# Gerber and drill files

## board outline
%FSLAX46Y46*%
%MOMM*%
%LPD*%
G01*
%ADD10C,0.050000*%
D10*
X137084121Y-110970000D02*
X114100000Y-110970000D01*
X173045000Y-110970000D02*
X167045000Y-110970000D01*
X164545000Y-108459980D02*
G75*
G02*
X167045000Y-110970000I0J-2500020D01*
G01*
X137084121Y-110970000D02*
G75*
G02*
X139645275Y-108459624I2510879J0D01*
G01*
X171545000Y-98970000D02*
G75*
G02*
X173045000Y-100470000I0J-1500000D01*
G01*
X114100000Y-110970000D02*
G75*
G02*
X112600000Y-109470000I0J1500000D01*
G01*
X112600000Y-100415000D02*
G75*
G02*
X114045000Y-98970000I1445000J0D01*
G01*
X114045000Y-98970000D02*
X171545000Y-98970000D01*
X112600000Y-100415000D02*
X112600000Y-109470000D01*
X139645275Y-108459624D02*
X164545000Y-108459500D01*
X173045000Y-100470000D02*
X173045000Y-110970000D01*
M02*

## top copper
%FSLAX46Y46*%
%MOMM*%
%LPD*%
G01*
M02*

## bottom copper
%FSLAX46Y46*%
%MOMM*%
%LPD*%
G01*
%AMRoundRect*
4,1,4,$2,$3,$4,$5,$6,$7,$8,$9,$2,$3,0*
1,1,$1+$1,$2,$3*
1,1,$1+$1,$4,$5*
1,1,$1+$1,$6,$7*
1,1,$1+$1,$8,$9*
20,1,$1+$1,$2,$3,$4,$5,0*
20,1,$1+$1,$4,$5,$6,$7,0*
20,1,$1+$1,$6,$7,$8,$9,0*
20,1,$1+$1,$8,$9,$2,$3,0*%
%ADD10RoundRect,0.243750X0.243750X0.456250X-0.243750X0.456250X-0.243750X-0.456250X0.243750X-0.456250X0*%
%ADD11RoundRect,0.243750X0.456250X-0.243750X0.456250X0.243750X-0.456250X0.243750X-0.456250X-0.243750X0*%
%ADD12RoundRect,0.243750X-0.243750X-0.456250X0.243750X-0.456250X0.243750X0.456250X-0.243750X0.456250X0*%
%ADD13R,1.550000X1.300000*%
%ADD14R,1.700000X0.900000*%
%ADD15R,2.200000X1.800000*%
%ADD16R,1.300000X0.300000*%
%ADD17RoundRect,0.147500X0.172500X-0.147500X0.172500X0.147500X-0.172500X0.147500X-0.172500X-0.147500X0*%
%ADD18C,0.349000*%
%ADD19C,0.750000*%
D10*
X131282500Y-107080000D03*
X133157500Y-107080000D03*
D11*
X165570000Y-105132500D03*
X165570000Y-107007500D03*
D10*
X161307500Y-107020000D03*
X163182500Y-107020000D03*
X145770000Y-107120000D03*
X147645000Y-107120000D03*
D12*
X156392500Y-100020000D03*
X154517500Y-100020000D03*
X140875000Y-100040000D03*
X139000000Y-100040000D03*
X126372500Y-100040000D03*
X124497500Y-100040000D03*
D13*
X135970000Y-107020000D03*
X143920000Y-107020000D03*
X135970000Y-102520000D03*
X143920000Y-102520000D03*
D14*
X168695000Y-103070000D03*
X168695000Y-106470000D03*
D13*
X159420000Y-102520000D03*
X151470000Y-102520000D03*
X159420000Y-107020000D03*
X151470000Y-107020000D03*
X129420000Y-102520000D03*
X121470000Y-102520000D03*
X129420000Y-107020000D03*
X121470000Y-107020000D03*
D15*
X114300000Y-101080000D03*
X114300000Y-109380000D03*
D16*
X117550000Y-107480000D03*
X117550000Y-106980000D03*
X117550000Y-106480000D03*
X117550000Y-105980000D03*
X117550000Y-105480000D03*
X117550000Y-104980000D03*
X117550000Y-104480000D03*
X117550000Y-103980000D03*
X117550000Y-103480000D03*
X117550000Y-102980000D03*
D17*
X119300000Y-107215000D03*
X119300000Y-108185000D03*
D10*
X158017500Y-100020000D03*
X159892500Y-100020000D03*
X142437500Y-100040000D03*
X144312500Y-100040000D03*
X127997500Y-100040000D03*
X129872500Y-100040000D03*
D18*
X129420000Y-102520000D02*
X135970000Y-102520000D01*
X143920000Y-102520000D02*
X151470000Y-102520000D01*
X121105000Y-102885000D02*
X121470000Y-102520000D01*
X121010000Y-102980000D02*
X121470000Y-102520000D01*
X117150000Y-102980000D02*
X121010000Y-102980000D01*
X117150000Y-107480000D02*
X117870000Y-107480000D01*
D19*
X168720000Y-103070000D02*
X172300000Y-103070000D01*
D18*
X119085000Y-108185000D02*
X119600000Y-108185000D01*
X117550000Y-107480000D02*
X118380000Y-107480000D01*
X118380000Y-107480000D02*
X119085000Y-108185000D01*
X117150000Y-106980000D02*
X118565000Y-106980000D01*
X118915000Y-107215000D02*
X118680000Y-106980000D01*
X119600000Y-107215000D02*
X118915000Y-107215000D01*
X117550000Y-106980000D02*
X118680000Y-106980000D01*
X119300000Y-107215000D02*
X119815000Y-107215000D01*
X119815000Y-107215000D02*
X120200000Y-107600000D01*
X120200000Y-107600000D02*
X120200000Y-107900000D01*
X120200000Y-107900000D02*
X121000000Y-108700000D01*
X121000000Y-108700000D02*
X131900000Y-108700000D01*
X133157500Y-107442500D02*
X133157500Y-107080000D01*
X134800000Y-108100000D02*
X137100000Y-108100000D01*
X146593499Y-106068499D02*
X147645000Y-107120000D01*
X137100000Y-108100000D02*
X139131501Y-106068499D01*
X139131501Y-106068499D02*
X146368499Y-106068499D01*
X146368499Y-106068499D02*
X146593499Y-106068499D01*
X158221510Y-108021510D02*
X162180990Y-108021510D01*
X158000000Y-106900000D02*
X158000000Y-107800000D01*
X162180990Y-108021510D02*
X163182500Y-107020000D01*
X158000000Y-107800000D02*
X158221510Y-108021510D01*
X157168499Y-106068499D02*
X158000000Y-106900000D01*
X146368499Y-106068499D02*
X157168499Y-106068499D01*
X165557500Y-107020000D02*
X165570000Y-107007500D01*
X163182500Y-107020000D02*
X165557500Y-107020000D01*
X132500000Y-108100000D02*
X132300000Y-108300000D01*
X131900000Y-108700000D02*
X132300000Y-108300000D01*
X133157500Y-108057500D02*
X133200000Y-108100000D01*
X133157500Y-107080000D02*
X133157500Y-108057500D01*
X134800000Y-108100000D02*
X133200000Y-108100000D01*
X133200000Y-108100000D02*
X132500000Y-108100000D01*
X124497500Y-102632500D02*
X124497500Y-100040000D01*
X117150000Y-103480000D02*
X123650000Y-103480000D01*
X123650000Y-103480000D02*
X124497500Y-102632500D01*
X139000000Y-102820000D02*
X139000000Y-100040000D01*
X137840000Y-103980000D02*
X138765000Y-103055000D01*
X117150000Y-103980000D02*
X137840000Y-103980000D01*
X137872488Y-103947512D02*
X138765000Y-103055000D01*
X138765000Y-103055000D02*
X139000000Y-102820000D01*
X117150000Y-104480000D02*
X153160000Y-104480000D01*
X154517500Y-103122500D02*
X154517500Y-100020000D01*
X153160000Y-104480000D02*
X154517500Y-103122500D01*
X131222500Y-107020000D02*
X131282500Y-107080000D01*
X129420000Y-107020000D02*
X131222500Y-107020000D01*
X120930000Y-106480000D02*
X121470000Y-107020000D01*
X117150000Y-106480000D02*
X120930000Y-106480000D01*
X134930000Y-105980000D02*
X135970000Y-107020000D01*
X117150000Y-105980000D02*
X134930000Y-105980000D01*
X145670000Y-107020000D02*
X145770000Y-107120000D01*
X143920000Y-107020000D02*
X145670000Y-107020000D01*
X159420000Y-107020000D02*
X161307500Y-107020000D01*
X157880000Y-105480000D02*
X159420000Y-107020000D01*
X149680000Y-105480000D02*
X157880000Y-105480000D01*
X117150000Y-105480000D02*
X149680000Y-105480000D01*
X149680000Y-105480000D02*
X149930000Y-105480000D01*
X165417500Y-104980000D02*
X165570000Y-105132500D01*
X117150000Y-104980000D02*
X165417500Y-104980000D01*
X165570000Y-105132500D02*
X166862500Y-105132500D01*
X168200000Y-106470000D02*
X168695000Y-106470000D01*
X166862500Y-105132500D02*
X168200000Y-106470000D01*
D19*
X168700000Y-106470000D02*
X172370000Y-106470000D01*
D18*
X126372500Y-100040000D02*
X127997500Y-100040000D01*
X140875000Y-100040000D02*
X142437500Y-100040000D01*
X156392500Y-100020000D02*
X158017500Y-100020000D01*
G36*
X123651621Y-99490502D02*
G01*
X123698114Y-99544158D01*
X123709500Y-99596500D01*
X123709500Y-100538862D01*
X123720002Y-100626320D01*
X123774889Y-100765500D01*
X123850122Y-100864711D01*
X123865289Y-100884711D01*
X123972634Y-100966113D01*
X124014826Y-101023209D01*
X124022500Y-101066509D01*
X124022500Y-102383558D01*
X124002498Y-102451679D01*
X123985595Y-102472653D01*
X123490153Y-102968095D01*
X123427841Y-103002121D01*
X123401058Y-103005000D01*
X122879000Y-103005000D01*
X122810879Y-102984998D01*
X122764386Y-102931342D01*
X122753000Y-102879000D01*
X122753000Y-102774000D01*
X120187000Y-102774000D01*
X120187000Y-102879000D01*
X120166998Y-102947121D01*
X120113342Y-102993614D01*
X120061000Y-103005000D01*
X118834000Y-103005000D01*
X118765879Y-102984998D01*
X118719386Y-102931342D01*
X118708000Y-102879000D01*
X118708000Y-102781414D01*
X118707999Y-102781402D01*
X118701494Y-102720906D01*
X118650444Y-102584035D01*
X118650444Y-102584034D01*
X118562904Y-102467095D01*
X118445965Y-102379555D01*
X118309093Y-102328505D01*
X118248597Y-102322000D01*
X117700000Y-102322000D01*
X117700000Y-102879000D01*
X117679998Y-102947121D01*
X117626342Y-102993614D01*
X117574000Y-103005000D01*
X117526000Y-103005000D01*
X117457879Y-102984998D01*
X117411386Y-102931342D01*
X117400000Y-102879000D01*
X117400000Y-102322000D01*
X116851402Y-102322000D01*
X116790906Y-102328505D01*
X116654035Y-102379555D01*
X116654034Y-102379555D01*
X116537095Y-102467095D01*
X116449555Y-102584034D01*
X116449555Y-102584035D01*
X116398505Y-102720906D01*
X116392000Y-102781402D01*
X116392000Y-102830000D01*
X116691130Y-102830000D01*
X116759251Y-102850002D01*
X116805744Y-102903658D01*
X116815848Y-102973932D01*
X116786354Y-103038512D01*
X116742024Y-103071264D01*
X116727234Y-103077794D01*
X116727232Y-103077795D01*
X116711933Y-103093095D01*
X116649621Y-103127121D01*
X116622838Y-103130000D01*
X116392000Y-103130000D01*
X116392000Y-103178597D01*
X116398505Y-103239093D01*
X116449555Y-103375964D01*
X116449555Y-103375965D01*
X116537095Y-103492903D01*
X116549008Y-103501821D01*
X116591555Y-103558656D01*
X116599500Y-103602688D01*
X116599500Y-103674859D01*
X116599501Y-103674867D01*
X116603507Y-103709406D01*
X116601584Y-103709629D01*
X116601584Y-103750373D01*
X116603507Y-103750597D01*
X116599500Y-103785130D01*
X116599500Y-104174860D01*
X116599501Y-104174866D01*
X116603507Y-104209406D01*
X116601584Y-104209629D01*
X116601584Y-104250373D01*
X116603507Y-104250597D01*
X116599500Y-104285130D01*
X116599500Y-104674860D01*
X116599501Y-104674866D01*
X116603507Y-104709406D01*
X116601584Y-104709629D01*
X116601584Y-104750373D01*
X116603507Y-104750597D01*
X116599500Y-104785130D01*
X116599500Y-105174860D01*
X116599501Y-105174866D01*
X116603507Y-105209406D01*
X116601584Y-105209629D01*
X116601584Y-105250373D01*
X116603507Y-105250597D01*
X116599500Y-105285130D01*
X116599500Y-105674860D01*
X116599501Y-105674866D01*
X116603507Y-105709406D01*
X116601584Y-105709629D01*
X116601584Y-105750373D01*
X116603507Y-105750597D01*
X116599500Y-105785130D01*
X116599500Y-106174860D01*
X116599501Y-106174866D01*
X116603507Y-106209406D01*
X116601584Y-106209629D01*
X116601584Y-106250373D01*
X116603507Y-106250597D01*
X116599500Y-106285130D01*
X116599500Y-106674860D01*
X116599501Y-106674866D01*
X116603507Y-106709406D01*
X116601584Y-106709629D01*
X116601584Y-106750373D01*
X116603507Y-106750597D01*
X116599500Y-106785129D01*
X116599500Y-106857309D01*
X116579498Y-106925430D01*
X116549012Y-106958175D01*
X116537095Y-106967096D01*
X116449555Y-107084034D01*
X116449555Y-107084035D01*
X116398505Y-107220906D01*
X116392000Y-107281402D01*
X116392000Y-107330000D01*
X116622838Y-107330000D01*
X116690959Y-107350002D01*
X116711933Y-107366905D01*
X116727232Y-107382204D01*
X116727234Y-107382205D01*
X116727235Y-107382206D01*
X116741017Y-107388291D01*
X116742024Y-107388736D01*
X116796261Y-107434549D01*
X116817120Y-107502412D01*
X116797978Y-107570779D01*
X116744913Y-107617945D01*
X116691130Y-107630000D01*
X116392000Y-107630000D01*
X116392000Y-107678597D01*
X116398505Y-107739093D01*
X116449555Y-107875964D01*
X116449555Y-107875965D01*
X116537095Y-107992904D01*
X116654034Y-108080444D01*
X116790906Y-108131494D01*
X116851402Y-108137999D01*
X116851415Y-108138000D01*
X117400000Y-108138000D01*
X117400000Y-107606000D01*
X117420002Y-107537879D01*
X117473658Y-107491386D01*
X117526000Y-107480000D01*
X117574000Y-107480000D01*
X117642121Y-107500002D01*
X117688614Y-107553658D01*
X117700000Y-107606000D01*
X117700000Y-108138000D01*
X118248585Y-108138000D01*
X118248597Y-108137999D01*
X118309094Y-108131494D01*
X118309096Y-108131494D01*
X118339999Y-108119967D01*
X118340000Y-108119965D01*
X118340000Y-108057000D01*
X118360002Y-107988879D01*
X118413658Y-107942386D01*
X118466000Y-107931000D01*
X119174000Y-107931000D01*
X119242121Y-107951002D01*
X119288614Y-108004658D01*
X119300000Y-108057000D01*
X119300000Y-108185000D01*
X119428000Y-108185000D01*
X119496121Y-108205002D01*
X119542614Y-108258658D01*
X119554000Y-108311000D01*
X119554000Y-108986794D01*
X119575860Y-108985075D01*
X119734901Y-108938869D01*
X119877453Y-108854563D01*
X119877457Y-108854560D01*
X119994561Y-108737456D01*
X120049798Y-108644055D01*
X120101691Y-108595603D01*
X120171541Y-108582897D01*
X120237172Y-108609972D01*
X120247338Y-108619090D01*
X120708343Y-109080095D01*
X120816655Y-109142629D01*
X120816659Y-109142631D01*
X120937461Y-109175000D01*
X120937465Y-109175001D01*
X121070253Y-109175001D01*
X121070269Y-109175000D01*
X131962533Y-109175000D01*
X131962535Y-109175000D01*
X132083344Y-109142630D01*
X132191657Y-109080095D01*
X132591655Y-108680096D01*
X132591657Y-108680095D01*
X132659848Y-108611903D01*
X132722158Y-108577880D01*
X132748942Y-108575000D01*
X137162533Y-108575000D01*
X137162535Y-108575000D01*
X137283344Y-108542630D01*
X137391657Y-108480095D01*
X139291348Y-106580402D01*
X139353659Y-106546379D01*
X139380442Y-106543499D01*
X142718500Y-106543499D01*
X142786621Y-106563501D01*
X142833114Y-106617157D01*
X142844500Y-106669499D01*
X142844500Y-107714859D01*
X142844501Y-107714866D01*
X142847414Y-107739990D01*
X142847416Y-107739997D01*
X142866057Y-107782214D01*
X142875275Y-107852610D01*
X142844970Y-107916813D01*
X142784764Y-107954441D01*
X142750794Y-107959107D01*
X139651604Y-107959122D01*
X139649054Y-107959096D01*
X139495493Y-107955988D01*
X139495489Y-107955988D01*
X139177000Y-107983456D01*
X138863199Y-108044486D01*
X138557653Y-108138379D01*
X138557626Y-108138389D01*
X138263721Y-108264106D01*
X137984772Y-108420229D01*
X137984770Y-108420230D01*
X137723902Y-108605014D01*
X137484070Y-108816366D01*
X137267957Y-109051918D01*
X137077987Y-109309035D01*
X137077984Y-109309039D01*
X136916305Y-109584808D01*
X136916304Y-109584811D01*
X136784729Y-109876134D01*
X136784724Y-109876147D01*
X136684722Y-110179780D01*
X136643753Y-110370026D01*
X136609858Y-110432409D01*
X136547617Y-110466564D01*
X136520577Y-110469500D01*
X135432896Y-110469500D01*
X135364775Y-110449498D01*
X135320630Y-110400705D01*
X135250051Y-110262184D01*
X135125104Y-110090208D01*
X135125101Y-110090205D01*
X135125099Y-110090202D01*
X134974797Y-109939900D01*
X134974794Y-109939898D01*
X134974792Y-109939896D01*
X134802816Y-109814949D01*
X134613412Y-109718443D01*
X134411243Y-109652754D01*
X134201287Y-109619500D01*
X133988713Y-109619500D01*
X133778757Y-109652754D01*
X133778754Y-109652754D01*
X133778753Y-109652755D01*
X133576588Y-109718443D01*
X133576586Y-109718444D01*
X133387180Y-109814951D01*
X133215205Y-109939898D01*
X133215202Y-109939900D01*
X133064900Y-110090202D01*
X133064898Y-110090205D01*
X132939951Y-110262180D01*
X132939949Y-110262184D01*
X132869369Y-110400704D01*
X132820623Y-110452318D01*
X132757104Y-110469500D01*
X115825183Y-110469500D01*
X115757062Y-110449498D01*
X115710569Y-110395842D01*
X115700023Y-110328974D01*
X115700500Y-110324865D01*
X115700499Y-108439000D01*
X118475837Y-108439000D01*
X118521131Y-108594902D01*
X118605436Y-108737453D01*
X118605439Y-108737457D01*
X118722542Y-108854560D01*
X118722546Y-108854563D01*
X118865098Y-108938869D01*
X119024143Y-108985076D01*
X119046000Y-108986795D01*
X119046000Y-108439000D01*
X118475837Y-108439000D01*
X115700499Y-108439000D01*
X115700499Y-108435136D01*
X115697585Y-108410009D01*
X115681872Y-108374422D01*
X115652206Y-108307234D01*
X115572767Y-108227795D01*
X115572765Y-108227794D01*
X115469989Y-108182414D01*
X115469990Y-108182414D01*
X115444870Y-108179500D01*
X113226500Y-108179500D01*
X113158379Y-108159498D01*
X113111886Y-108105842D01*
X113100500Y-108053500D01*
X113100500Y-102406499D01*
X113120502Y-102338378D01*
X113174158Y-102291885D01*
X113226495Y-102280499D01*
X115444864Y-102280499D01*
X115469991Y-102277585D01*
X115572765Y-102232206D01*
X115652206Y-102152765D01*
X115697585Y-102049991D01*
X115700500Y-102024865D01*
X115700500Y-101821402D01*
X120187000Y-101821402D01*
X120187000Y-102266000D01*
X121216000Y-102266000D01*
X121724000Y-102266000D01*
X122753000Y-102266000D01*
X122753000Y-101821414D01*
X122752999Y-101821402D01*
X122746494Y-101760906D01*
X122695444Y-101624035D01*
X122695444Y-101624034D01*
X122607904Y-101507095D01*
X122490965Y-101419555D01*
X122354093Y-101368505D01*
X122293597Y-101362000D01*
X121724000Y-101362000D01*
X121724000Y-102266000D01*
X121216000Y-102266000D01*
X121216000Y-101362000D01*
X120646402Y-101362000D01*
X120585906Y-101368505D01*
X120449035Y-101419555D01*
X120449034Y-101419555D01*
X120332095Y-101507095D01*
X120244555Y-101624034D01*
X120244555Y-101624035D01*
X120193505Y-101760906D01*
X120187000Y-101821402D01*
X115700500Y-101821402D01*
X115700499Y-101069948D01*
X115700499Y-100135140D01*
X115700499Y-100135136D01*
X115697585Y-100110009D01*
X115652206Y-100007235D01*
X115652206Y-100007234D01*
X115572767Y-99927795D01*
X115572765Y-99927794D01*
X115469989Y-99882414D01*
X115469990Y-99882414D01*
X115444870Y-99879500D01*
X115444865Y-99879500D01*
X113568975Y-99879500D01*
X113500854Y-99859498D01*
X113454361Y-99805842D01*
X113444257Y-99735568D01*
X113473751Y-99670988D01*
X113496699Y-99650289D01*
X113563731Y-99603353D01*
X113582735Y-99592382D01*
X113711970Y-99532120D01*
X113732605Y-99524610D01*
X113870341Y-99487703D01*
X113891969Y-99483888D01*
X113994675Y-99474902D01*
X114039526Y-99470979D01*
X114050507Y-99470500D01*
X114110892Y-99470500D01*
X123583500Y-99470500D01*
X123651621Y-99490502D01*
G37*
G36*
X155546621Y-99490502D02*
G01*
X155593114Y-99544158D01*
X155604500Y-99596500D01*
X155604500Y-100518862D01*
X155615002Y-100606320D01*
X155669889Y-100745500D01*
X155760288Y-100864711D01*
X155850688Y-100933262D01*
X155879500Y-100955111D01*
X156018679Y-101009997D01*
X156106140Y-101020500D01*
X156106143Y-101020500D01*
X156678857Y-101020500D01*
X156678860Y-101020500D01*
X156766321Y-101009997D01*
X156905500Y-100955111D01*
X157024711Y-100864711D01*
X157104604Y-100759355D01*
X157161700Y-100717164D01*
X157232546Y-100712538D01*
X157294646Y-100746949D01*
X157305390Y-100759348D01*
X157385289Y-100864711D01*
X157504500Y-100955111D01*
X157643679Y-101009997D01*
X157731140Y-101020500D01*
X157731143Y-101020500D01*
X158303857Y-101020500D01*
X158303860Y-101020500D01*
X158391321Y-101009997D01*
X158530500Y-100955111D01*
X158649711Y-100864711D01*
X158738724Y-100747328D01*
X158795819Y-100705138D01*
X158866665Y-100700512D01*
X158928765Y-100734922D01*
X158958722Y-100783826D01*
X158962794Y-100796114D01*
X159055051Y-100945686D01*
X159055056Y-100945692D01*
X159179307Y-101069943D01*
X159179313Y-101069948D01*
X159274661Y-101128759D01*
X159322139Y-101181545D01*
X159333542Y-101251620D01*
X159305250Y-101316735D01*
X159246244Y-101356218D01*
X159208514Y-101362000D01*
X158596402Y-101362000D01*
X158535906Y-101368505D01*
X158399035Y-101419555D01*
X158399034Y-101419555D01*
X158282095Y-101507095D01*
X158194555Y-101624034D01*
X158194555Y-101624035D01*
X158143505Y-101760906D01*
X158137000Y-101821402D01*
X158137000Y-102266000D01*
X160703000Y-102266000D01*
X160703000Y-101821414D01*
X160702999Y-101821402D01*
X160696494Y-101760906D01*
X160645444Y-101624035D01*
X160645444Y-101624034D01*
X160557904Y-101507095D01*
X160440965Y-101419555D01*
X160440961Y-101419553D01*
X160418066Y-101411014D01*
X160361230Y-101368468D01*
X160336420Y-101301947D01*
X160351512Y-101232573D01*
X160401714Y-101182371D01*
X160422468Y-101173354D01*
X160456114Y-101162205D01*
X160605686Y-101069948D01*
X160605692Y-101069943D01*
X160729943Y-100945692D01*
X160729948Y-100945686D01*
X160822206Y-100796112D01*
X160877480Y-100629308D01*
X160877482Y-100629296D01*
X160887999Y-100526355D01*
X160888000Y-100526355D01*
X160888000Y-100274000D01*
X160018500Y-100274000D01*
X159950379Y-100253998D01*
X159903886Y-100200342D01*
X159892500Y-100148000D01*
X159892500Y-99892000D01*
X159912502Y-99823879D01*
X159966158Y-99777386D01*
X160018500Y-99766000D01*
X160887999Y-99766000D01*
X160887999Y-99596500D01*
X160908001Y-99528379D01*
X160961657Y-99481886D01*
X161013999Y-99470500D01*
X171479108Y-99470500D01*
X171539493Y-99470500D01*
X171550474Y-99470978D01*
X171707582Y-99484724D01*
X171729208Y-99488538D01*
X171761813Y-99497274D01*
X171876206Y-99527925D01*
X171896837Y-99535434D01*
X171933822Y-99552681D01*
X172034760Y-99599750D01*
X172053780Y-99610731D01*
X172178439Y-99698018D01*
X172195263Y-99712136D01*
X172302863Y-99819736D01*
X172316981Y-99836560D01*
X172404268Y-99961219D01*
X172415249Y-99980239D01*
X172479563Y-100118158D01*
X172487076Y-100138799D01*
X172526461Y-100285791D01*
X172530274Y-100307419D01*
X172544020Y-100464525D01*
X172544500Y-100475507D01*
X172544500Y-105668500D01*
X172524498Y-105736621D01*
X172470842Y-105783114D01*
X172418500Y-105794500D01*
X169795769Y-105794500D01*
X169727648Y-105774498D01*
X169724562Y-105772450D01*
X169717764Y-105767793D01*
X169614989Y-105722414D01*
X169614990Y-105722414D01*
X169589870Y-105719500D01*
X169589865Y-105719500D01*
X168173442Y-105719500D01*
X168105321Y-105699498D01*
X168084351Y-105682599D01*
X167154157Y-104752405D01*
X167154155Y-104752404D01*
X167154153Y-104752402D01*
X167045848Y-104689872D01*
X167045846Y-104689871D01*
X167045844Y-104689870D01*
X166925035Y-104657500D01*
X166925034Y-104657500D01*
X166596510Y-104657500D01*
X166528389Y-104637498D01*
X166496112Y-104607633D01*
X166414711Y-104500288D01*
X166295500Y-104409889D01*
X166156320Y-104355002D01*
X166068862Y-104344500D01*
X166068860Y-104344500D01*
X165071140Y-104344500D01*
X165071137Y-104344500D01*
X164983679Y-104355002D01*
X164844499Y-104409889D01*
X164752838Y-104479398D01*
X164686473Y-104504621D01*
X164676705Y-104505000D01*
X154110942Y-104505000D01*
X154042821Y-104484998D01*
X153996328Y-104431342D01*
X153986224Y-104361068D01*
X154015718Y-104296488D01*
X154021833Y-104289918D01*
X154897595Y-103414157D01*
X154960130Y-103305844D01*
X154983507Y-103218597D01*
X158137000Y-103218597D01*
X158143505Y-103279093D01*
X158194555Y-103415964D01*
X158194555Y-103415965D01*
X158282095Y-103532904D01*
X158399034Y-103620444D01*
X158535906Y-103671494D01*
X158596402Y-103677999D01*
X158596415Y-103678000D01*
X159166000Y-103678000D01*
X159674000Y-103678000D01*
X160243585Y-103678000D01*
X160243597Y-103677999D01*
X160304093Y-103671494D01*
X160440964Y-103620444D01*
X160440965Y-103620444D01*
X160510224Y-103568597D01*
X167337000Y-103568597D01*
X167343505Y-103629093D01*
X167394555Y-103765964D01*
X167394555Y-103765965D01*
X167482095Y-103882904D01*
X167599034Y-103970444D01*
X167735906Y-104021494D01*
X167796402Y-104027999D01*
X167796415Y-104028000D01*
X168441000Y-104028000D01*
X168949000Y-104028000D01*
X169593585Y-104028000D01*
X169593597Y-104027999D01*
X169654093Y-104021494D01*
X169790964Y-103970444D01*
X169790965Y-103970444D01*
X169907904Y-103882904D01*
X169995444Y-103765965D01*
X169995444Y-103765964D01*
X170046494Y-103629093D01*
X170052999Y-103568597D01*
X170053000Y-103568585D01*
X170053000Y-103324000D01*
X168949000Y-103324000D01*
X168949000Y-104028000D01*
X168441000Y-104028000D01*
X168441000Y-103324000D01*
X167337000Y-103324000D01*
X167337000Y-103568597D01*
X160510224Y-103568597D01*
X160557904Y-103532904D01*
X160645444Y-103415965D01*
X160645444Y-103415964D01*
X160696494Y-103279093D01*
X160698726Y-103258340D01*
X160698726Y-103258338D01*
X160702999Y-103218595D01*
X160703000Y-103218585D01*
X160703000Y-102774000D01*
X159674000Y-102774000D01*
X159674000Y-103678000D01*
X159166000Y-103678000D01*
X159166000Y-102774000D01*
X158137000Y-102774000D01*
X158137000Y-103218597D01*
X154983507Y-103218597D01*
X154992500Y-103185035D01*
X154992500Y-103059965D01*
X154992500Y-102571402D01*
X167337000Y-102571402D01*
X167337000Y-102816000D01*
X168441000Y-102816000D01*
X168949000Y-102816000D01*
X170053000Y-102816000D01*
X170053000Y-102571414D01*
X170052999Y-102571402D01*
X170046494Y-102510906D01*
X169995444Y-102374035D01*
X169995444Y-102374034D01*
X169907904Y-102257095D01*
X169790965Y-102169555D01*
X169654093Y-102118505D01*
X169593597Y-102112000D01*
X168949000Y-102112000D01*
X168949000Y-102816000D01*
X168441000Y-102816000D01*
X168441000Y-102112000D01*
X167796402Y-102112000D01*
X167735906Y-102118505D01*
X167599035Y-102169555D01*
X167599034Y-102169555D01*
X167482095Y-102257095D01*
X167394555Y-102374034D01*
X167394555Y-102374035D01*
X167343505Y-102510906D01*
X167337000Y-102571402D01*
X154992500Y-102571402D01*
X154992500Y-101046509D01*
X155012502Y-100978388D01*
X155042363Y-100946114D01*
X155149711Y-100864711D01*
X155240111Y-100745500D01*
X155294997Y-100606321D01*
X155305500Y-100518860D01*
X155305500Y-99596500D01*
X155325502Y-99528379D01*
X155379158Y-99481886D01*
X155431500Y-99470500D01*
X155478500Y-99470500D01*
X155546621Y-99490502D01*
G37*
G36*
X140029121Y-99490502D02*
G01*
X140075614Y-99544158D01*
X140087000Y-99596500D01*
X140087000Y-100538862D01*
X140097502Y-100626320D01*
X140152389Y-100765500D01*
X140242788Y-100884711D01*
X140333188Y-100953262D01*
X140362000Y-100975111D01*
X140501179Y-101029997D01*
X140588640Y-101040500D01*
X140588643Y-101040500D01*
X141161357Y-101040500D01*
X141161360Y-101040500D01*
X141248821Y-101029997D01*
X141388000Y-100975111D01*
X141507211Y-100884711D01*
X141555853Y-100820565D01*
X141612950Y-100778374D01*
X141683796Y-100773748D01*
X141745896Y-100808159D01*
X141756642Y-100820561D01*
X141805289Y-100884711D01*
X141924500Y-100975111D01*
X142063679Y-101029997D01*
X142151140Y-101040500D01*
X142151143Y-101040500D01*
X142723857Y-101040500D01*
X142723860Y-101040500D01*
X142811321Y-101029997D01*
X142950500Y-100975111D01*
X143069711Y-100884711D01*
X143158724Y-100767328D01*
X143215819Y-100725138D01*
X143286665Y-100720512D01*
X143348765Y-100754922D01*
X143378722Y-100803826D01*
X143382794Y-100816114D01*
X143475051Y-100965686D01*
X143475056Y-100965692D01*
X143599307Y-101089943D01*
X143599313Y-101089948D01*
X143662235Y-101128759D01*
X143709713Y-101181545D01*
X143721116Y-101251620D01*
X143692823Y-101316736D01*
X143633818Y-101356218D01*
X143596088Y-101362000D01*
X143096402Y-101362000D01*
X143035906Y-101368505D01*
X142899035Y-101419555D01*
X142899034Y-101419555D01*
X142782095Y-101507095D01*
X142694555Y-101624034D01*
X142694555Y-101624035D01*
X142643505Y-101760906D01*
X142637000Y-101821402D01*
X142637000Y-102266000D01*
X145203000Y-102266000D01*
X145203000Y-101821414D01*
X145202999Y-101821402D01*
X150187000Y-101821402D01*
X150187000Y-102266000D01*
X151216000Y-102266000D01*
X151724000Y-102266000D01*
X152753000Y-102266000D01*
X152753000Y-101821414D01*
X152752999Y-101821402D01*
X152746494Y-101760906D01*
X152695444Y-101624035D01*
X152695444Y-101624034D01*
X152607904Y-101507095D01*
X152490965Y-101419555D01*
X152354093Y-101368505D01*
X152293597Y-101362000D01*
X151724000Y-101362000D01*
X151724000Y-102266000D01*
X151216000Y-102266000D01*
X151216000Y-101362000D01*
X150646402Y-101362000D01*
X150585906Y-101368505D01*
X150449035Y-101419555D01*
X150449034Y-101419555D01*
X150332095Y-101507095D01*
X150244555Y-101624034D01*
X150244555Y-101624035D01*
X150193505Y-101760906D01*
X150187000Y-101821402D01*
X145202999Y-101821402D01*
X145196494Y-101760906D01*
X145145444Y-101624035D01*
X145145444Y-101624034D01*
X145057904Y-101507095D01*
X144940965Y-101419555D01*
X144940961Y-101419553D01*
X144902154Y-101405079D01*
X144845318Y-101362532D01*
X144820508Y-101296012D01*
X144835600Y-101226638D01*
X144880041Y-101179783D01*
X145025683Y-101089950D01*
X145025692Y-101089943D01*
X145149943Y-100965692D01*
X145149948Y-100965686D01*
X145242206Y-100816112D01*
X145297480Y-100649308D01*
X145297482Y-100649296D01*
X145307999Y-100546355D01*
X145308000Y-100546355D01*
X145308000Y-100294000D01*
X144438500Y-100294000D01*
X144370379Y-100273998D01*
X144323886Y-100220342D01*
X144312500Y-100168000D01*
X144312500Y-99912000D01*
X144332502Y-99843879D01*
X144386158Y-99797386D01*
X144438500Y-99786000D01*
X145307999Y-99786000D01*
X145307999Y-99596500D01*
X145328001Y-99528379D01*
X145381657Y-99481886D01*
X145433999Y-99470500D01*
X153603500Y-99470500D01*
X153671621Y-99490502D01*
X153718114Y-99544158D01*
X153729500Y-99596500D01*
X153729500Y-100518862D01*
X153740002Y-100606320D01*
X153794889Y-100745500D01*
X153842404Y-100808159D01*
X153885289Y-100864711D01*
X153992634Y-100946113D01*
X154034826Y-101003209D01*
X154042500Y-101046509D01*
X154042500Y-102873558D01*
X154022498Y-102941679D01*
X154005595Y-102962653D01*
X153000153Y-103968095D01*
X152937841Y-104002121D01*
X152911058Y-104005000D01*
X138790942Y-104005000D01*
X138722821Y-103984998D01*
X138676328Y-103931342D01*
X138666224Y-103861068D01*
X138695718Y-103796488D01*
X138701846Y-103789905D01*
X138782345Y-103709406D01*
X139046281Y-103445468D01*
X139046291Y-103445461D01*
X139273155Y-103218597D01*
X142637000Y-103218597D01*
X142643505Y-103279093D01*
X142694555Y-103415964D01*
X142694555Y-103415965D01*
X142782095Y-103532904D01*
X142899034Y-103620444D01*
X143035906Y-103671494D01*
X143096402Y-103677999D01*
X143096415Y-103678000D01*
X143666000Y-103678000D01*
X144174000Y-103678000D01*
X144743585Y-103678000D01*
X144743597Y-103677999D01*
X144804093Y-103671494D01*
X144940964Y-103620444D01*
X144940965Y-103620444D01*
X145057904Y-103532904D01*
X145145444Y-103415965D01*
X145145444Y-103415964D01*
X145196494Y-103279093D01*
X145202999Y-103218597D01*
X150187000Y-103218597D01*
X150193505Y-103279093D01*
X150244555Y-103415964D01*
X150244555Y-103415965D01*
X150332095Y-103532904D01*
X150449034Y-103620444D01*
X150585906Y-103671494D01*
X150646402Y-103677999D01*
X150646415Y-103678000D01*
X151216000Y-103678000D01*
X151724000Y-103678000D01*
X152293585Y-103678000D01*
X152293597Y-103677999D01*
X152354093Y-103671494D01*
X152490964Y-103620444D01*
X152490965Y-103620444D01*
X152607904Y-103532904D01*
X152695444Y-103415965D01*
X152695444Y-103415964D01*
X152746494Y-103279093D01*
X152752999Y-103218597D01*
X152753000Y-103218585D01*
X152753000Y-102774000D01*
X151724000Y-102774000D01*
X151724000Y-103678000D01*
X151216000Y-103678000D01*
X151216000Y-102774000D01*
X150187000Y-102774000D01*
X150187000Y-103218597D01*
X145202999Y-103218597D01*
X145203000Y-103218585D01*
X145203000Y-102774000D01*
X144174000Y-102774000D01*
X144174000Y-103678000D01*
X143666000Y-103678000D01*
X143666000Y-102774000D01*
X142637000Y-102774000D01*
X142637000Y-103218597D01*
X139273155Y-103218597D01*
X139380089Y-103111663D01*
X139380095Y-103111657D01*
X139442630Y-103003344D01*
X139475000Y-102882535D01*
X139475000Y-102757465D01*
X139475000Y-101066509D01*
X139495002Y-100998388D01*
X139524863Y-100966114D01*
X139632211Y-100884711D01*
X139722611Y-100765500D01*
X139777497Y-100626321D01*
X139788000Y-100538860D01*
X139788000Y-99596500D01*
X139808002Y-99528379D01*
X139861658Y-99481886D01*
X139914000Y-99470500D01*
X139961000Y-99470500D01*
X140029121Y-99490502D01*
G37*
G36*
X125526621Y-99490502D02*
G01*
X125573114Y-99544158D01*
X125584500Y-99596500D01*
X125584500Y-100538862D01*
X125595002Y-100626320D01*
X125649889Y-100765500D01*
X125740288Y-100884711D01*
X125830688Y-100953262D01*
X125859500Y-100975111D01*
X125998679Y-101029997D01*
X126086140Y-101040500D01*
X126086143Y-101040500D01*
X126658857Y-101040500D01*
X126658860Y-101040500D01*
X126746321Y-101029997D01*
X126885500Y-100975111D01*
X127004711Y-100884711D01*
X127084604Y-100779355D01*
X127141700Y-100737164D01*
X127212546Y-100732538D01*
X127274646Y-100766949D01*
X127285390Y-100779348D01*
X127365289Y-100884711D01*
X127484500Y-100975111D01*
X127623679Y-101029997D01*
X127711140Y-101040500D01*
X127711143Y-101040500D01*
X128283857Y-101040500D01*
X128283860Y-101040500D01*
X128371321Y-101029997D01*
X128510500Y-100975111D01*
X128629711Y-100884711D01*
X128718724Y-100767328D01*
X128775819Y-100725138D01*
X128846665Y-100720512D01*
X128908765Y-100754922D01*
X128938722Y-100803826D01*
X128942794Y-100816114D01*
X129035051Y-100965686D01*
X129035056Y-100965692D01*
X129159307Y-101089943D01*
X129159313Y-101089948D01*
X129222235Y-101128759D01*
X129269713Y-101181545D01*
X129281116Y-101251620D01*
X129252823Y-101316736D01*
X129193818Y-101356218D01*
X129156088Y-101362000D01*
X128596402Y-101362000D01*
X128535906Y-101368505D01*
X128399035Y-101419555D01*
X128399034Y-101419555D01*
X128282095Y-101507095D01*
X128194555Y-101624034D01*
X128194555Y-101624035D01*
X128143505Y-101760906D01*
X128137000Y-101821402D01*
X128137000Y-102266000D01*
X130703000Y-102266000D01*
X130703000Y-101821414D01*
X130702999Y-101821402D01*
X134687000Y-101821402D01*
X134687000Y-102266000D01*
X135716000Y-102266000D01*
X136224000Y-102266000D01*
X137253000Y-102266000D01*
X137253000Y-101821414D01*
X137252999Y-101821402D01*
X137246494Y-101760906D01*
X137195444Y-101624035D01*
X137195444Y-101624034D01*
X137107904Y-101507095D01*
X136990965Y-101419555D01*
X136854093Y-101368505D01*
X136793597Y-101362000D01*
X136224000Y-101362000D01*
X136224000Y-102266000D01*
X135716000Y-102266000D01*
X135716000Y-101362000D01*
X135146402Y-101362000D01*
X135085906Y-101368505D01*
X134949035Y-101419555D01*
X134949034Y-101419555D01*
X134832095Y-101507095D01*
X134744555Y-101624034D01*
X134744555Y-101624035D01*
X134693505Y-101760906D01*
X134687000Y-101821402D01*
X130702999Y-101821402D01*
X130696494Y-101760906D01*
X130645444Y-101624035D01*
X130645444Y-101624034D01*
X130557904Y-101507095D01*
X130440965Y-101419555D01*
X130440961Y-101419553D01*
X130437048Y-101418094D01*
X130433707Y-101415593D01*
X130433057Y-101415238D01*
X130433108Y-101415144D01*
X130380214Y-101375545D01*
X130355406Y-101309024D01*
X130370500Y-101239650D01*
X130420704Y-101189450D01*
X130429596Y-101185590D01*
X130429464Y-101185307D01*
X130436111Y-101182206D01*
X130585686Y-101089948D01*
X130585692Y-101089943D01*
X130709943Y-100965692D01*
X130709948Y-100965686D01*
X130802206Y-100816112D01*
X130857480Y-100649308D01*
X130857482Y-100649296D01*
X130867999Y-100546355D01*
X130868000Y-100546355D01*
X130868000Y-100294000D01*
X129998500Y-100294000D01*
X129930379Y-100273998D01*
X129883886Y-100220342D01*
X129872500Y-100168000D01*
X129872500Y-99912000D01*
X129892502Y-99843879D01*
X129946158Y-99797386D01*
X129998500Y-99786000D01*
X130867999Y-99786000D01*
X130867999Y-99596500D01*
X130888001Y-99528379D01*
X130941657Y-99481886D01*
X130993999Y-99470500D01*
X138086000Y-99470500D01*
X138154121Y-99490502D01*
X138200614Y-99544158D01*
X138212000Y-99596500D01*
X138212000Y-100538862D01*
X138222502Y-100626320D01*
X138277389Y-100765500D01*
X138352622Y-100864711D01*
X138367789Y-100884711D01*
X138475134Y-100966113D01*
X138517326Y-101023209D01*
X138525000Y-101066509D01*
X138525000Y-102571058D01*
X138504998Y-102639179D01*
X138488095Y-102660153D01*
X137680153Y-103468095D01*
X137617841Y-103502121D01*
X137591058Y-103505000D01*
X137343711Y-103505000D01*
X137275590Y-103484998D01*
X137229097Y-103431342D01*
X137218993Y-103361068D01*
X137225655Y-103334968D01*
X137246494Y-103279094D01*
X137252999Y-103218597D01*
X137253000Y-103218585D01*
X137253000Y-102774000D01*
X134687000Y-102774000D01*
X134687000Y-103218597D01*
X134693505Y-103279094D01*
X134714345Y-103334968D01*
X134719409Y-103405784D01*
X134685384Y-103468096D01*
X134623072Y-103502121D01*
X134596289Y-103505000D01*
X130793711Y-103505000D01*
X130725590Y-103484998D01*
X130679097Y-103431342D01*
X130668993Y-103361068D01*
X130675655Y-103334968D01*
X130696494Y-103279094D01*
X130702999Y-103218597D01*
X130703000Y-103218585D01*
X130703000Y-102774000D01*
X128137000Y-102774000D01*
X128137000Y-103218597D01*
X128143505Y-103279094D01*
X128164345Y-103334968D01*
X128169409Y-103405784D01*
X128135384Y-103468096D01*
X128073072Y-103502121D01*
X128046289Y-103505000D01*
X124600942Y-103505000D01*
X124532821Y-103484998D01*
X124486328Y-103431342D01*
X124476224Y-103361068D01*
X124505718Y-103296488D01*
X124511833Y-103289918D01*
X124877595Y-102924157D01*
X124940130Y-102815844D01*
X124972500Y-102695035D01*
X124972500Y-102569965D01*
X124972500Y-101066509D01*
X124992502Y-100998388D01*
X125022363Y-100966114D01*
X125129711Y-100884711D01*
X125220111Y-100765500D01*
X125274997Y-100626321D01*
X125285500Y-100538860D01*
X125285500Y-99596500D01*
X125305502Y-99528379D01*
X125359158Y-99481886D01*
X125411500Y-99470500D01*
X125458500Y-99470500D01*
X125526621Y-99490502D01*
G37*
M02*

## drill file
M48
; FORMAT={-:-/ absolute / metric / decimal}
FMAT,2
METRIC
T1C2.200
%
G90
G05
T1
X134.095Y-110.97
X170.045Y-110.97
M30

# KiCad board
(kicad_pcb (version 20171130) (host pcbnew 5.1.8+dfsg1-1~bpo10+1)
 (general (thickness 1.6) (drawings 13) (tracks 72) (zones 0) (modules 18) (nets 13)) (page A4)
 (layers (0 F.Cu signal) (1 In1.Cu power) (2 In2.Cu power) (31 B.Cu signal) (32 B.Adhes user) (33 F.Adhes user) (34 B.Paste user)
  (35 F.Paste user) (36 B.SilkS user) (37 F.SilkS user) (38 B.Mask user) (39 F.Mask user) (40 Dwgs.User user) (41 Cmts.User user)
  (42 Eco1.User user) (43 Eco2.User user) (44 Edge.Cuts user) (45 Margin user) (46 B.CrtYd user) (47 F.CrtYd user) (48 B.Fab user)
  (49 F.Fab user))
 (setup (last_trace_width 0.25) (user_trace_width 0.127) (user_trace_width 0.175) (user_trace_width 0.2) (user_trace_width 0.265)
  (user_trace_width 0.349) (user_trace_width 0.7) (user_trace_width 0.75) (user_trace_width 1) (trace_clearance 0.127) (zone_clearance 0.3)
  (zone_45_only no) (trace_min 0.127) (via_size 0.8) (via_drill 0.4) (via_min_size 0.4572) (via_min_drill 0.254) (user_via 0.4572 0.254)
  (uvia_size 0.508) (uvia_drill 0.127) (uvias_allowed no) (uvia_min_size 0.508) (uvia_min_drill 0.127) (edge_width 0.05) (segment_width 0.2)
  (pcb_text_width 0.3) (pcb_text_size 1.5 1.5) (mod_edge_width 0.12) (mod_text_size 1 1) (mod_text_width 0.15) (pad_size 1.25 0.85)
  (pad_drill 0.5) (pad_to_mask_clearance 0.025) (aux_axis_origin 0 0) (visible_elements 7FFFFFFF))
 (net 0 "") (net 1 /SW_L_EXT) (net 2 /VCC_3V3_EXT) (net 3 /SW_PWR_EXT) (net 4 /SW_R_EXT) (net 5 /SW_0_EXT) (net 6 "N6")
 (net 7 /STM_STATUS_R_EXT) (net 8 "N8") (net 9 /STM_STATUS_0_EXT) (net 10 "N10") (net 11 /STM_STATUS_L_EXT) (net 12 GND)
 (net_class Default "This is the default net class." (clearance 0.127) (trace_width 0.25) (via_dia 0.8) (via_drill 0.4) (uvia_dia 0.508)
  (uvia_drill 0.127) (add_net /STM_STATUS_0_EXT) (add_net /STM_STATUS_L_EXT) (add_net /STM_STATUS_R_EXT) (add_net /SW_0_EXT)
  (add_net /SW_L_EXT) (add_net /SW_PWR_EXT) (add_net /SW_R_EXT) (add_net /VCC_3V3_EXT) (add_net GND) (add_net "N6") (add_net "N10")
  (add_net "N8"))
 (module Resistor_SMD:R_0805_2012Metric (layer B.Cu) (at 132.22 107.08 180)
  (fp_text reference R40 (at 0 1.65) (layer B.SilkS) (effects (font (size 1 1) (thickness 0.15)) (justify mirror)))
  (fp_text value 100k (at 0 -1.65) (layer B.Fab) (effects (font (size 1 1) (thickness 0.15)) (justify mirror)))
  (pad 2 smd roundrect (at 0.9375 0 180) (size 0.975 1.4) (layers B.Cu B.Paste B.Mask) (roundrect_rratio 0.25) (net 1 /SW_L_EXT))
  (pad 1 smd roundrect (at -0.9375 0 180) (size 0.975 1.4) (layers B.Cu B.Paste B.Mask) (roundrect_rratio 0.25) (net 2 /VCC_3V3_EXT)))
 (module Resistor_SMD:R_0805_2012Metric (layer B.Cu) (at 165.57 106.07 90)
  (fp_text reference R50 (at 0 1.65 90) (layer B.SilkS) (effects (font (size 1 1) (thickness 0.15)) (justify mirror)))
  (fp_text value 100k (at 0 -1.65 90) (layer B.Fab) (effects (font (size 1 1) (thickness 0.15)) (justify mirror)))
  (pad 2 smd roundrect (at 0.9375 0 90) (size 0.975 1.4) (layers B.Cu B.Paste B.Mask) (roundrect_rratio 0.25) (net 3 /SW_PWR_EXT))
  (pad 1 smd roundrect (at -0.9375 0 90) (size 0.975 1.4) (layers B.Cu B.Paste B.Mask) (roundrect_rratio 0.25) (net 2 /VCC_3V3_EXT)))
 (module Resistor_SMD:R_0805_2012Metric (layer B.Cu) (at 162.245 107.02 180)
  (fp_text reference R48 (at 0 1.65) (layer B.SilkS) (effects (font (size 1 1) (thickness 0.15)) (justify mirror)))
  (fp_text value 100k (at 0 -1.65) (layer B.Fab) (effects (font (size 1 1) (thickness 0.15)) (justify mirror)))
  (pad 2 smd roundrect (at 0.9375 0 180) (size 0.975 1.4) (layers B.Cu B.Paste B.Mask) (roundrect_rratio 0.25) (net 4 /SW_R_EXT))
  (pad 1 smd roundrect (at -0.9375 0 180) (size 0.975 1.4) (layers B.Cu B.Paste B.Mask) (roundrect_rratio 0.25) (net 2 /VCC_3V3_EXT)))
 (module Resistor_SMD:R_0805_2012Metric (layer B.Cu) (at 146.7075 107.12 180)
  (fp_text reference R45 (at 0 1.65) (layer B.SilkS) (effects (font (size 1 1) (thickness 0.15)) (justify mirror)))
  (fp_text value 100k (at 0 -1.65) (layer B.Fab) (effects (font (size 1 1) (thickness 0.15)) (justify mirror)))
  (pad 2 smd roundrect (at 0.9375 0 180) (size 0.975 1.4) (layers B.Cu B.Paste B.Mask) (roundrect_rratio 0.25) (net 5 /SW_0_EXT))
  (pad 1 smd roundrect (at -0.9375 0 180) (size 0.975 1.4) (layers B.Cu B.Paste B.Mask) (roundrect_rratio 0.25) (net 2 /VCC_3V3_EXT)))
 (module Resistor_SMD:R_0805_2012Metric (layer B.Cu) (at 155.455 100.02)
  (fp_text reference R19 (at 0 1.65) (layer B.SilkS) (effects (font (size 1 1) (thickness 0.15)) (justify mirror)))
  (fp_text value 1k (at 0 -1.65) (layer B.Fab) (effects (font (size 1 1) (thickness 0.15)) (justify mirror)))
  (pad 2 smd roundrect (at 0.9375 0) (size 0.975 1.4) (layers B.Cu B.Paste B.Mask) (roundrect_rratio 0.25) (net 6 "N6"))
  (pad 1 smd roundrect (at -0.9375 0) (size 0.975 1.4) (layers B.Cu B.Paste B.Mask) (roundrect_rratio 0.25) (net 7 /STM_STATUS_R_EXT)))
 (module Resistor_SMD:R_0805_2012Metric (layer B.Cu) (at 139.9375 100.04)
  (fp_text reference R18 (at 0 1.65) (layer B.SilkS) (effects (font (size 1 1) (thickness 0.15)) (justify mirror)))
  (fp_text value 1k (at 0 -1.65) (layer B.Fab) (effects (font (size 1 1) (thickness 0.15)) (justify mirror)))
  (pad 2 smd roundrect (at 0.9375 0) (size 0.975 1.4) (layers B.Cu B.Paste B.Mask) (roundrect_rratio 0.25) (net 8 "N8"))
  (pad 1 smd roundrect (at -0.9375 0) (size 0.975 1.4) (layers B.Cu B.Paste B.Mask) (roundrect_rratio 0.25) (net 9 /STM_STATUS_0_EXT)))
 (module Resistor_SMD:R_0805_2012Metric (layer B.Cu) (at 125.435 100.04)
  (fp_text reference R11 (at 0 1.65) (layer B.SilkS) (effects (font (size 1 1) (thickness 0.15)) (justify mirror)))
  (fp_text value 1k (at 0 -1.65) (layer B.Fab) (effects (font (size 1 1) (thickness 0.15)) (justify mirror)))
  (pad 2 smd roundrect (at 0.9375 0) (size 0.975 1.4) (layers B.Cu B.Paste B.Mask) (roundrect_rratio 0.25) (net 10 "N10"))
  (pad 1 smd roundrect (at -0.9375 0) (size 0.975 1.4) (layers B.Cu B.Paste B.Mask) (roundrect_rratio 0.25) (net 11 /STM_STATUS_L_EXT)))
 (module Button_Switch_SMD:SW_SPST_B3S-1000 (layer B.Cu) (at 139.945 104.77)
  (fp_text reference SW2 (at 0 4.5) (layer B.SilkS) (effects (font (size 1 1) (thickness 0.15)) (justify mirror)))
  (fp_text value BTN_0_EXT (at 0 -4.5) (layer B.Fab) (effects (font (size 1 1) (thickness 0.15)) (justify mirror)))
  (pad 1 smd rect (at -3.975 2.25) (size 1.55 1.3) (layers B.Cu B.Paste B.Mask) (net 5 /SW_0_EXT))
  (pad 1 smd rect (at 3.975 2.25) (size 1.55 1.3) (layers B.Cu B.Paste B.Mask) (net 5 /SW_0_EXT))
  (pad 2 smd rect (at -3.975 -2.25) (size 1.55 1.3) (layers B.Cu B.Paste B.Mask) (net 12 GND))
  (pad 2 smd rect (at 3.975 -2.25) (size 1.55 1.3) (layers B.Cu B.Paste B.Mask) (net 12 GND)))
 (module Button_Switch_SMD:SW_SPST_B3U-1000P (layer B.Cu) (at 168.695 104.77 90)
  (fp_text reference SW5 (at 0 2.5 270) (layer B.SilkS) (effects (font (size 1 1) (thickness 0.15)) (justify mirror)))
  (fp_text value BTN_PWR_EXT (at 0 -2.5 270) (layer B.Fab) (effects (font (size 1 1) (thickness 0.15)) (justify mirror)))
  (pad 2 smd rect (at 1.7 0 90) (size 0.9 1.7) (layers B.Cu B.Paste B.Mask) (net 12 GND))
  (pad 1 smd rect (at -1.7 0 90) (size 0.9 1.7) (layers B.Cu B.Paste B.Mask) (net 3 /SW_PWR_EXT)))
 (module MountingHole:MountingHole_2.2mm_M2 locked (layer F.Cu) (at 134.095 110.97 180)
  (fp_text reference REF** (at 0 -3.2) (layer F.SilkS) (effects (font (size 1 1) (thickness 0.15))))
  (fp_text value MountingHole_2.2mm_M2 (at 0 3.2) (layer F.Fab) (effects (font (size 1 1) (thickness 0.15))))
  (pad 1 np_thru_hole circle (at 0 0 180) (size 2.2 2.2) (drill 2.2) (layers *.Cu *.Mask)))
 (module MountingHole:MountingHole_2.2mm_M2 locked (layer F.Cu) (at 170.045 110.97 270)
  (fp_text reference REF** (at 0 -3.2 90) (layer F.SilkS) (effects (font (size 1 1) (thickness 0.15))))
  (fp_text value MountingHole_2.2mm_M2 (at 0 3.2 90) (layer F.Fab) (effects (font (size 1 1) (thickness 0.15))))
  (pad 1 np_thru_hole circle (at 0 0 270) (size 2.2 2.2) (drill 2.2) (layers *.Cu *.Mask)))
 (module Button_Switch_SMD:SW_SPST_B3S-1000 (layer B.Cu) (at 155.445 104.77)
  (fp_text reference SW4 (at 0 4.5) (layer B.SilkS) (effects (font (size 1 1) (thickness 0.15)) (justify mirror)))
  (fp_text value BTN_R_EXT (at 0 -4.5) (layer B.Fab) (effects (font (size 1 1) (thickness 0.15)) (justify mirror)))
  (pad 2 smd rect (at 3.975 -2.25) (size 1.55 1.3) (layers B.Cu B.Paste B.Mask) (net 12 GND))
  (pad 2 smd rect (at -3.975 -2.25) (size 1.55 1.3) (layers B.Cu B.Paste B.Mask) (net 12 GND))
  (pad 1 smd rect (at 3.975 2.25) (size 1.55 1.3) (layers B.Cu B.Paste B.Mask) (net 4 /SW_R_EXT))
  (pad 1 smd rect (at -3.975 2.25) (size 1.55 1.3) (layers B.Cu B.Paste B.Mask) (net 4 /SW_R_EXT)))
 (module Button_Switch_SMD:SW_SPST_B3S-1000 (layer B.Cu) (at 125.445 104.77)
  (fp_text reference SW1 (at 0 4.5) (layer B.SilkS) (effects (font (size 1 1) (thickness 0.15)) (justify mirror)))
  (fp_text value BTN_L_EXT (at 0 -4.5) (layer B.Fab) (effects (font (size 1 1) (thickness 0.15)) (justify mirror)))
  (pad 2 smd rect (at 3.975 -2.25) (size 1.55 1.3) (layers B.Cu B.Paste B.Mask) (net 12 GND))
  (pad 2 smd rect (at -3.975 -2.25) (size 1.55 1.3) (layers B.Cu B.Paste B.Mask) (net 12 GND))
  (pad 1 smd rect (at 3.975 2.25) (size 1.55 1.3) (layers B.Cu B.Paste B.Mask) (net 1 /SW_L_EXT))
  (pad 1 smd rect (at -3.975 2.25) (size 1.55 1.3) (layers B.Cu B.Paste B.Mask) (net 1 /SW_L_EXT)))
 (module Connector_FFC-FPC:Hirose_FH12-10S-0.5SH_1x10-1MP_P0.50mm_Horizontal (layer B.Cu) (at 115.7 105.23 90)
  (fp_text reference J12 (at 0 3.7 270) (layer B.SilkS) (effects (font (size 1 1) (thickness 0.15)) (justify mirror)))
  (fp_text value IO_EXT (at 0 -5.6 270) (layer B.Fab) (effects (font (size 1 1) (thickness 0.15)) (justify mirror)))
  (pad MP smd rect (at 4.15 -1.4 90) (size 1.8 2.2) (layers B.Cu B.Paste B.Mask))
  (pad MP smd rect (at -4.15 -1.4 90) (size 1.8 2.2) (layers B.Cu B.Paste B.Mask))
  (pad 1 smd rect (at -2.25 1.85 90) (size 0.3 1.3) (layers B.Cu B.Paste B.Mask) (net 12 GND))
  (pad 2 smd rect (at -1.75 1.85 90) (size 0.3 1.3) (layers B.Cu B.Paste B.Mask) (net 2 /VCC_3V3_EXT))
  (pad 3 smd rect (at -1.25 1.85 90) (size 0.3 1.3) (layers B.Cu B.Paste B.Mask) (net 1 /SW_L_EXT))
  (pad 4 smd rect (at -0.75 1.85 90) (size 0.3 1.3) (layers B.Cu B.Paste B.Mask) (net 5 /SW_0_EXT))
  (pad 5 smd rect (at -0.25 1.85 90) (size 0.3 1.3) (layers B.Cu B.Paste B.Mask) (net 4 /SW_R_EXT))
  (pad 6 smd rect (at 0.25 1.85 90) (size 0.3 1.3) (layers B.Cu B.Paste B.Mask) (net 3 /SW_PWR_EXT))
  (pad 7 smd rect (at 0.75 1.85 90) (size 0.3 1.3) (layers B.Cu B.Paste B.Mask) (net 7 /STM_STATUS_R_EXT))
  (pad 8 smd rect (at 1.25 1.85 90) (size 0.3 1.3) (layers B.Cu B.Paste B.Mask) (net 9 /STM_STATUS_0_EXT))
  (pad 9 smd rect (at 1.75 1.85 90) (size 0.3 1.3) (layers B.Cu B.Paste B.Mask) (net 11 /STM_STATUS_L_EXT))
  (pad 10 smd rect (at 2.25 1.85 90) (size 0.3 1.3) (layers B.Cu B.Paste B.Mask) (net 12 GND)))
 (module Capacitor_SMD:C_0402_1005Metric (layer B.Cu) (at 119.3 107.7 90)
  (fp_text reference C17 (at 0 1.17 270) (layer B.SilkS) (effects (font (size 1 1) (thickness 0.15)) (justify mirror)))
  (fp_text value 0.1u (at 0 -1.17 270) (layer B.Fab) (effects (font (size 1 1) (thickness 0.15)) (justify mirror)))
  (pad 2 smd roundrect (at 0.485 0 90) (size 0.59 0.64) (layers B.Cu B.Paste B.Mask) (roundrect_rratio 0.25) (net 2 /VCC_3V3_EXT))
  (pad 1 smd roundrect (at -0.485 0 90) (size 0.59 0.64) (layers B.Cu B.Paste B.Mask) (roundrect_rratio 0.25) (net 12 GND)))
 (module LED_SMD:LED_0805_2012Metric (layer B.Cu) (at 158.955 100.02 180)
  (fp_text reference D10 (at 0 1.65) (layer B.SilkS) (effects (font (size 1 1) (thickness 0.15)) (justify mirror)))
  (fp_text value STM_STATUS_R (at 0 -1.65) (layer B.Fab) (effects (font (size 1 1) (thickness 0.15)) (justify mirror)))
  (pad 2 smd roundrect (at 0.9375 0 180) (size 0.975 1.4) (layers B.Cu B.Paste B.Mask) (roundrect_rratio 0.25) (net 6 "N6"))
  (pad 1 smd roundrect (at -0.9375 0 180) (size 0.975 1.4) (layers B.Cu B.Paste B.Mask) (roundrect_rratio 0.25) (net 12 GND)))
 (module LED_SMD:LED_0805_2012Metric (layer B.Cu) (at 143.375 100.04 180)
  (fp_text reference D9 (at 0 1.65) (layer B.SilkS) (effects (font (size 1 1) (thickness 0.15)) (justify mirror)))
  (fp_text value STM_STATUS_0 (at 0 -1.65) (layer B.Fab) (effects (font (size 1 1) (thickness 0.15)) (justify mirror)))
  (pad 2 smd roundrect (at 0.9375 0 180) (size 0.975 1.4) (layers B.Cu B.Paste B.Mask) (roundrect_rratio 0.25) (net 8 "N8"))
  (pad 1 smd roundrect (at -0.9375 0 180) (size 0.975 1.4) (layers B.Cu B.Paste B.Mask) (roundrect_rratio 0.25) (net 12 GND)))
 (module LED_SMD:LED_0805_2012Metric (layer B.Cu) (at 128.935 100.04 180)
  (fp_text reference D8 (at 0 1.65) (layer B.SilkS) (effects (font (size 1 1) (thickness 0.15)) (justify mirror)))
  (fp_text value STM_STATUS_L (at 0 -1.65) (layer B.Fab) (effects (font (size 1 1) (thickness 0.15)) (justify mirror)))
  (pad 2 smd roundrect (at 0.9375 0 180) (size 0.975 1.4) (layers B.Cu B.Paste B.Mask) (roundrect_rratio 0.25) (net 10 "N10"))
  (pad 1 smd roundrect (at -0.9375 0 180) (size 0.975 1.4) (layers B.Cu B.Paste B.Mask) (roundrect_rratio 0.25) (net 12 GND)))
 (gr_line (start 137.084121 110.97) (end 114.1 110.97) (layer Edge.Cuts) (width 0.05))
 (gr_line (start 173.045 110.97) (end 167.045 110.97) (layer Edge.Cuts) (width 0.05))
 (gr_arc (start 164.545 110.96) (end 167.045 110.97) (angle -90.2291819) (layer Edge.Cuts) (width 0.05))
 (gr_arc (start 139.595 110.97) (end 137.084121 110.97) (angle 91.14730236) (layer Edge.Cuts) (width 0.05))
 (gr_arc (start 171.545 100.47) (end 173.045 100.47) (angle -90) (layer Edge.Cuts) (width 0.05))
 (gr_arc (start 114.1 109.47) (end 114.1 110.97) (angle 90) (layer Edge.Cuts) (width 0.05))
 (gr_arc (start 114.045 100.415) (end 112.6 100.415) (angle 90) (layer Edge.Cuts) (width 0.05))
 (gr_line (start 114.045 98.97) (end 171.545 98.97) (layer Edge.Cuts) (width 0.05))
 (gr_line (start 112.6 100.415) (end 112.6 109.47) (layer Edge.Cuts) (width 0.05))
 (gr_line (start 139.645275 108.459624) (end 164.545 108.4595) (layer Edge.Cuts) (width 0.05))
 (gr_line (start 173.045 100.47) (end 173.045 110.97) (layer Edge.Cuts) (width 0.05))
 (segment (start 129.42 102.52) (end 135.97 102.52) (width 0.349) (layer B.Cu) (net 12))
 (segment (start 143.92 102.52) (end 151.47 102.52) (width 0.349) (layer B.Cu) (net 12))
 (segment (start 121.105 102.885) (end 121.47 102.52) (width 0.349) (layer B.Cu) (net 12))
 (segment (start 121.01 102.98) (end 121.47 102.52) (width 0.349) (layer B.Cu) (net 12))
 (segment (start 117.15 102.98) (end 121.01 102.98) (width 0.349) (layer B.Cu) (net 12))
 (segment (start 117.15 107.48) (end 117.87 107.48) (width 0.349) (layer B.Cu) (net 12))
 (segment (start 168.72 103.07) (end 172.3 103.07) (width 0.75) (layer B.Cu) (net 12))
 (segment (start 119.085 108.185) (end 119.6 108.185) (width 0.349) (layer B.Cu) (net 12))
 (segment (start 117.55 107.48) (end 118.38 107.48) (width 0.349) (layer B.Cu) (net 12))
 (segment (start 118.38 107.48) (end 119.085 108.185) (width 0.349) (layer B.Cu) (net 12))
 (segment (start 117.15 106.98) (end 118.565 106.98) (width 0.349) (layer B.Cu) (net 2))
 (segment (start 118.915 107.215) (end 118.68 106.98) (width 0.349) (layer B.Cu) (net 2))
 (segment (start 119.6 107.215) (end 118.915 107.215) (width 0.349) (layer B.Cu) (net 2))
 (segment (start 117.55 106.98) (end 118.68 106.98) (width 0.349) (layer B.Cu) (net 2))
 (segment (start 119.3 107.215) (end 119.815 107.215) (width 0.349) (layer B.Cu) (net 2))
 (segment (start 119.815 107.215) (end 120.2 107.6) (width 0.349) (layer B.Cu) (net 2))
 (segment (start 120.2 107.6) (end 120.2 107.9) (width 0.349) (layer B.Cu) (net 2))
 (segment (start 120.2 107.9) (end 121 108.7) (width 0.349) (layer B.Cu) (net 2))
 (segment (start 121 108.7) (end 131.9 108.7) (width 0.349) (layer B.Cu) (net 2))
 (segment (start 133.1575 107.4425) (end 133.1575 107.08) (width 0.349) (layer B.Cu) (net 2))
 (segment (start 134.8 108.1) (end 137.1 108.1) (width 0.349) (layer B.Cu) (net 2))
 (segment (start 146.593499 106.068499) (end 147.645 107.12) (width 0.349) (layer B.Cu) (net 2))
 (segment (start 137.1 108.1) (end 139.131501 106.068499) (width 0.349) (layer B.Cu) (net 2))
 (segment (start 139.131501 106.068499) (end 146.368499 106.068499) (width 0.349) (layer B.Cu) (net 2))
 (segment (start 146.368499 106.068499) (end 146.593499 106.068499) (width 0.349) (layer B.Cu) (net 2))
 (segment (start 158.22151 108.02151) (end 162.18099 108.02151) (width 0.349) (layer B.Cu) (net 2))
 (segment (start 158 106.9) (end 158 107.8) (width 0.349) (layer B.Cu) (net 2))
 (segment (start 162.18099 108.02151) (end 163.1825 107.02) (width 0.349) (layer B.Cu) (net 2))
 (segment (start 158 107.8) (end 158.22151 108.02151) (width 0.349) (layer B.Cu) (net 2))
 (segment (start 157.168499 106.068499) (end 158 106.9) (width 0.349) (layer B.Cu) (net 2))
 (segment (start 146.368499 106.068499) (end 157.168499 106.068499) (width 0.349) (layer B.Cu) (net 2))
 (segment (start 165.5575 107.02) (end 165.57 107.0075) (width 0.349) (layer B.Cu) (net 2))
 (segment (start 163.1825 107.02) (end 165.5575 107.02) (width 0.349) (layer B.Cu) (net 2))
 (segment (start 132.5 108.1) (end 132.3 108.3) (width 0.349) (layer B.Cu) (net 2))
 (segment (start 131.9 108.7) (end 132.3 108.3) (width 0.349) (layer B.Cu) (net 2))
 (segment (start 133.1575 108.0575) (end 133.2 108.1) (width 0.349) (layer B.Cu) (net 2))
 (segment (start 133.1575 107.08) (end 133.1575 108.0575) (width 0.349) (layer B.Cu) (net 2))
 (segment (start 134.8 108.1) (end 133.2 108.1) (width 0.349) (layer B.Cu) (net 2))
 (segment (start 133.2 108.1) (end 132.5 108.1) (width 0.349) (layer B.Cu) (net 2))
 (segment (start 124.4975 102.6325) (end 124.4975 100.04) (width 0.349) (layer B.Cu) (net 11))
 (segment (start 117.15 103.48) (end 123.65 103.48) (width 0.349) (layer B.Cu) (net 11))
 (segment (start 123.65 103.48) (end 124.4975 102.6325) (width 0.349) (layer B.Cu) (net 11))
 (segment (start 139 102.82) (end 139 100.04) (width 0.349) (layer B.Cu) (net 9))
 (segment (start 137.84 103.98) (end 138.765 103.055) (width 0.349) (layer B.Cu) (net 9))
 (segment (start 117.15 103.98) (end 137.84 103.98) (width 0.349) (layer B.Cu) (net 9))
 (segment (start 137.872488 103.947512) (end 138.765 103.055) (width 0.349) (layer B.Cu) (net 9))
 (segment (start 138.765 103.055) (end 139 102.82) (width 0.349) (layer B.Cu) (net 9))
 (segment (start 117.15 104.48) (end 153.16 104.48) (width 0.349) (layer B.Cu) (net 7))
 (segment (start 154.5175 103.1225) (end 154.5175 100.02) (width 0.349) (layer B.Cu) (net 7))
 (segment (start 153.16 104.48) (end 154.5175 103.1225) (width 0.349) (layer B.Cu) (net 7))
 (segment (start 131.2225 107.02) (end 131.2825 107.08) (width 0.349) (layer B.Cu) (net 1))
 (segment (start 129.42 107.02) (end 131.2225 107.02) (width 0.349) (layer B.Cu) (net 1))
 (segment (start 120.93 106.48) (end 121.47 107.02) (width 0.349) (layer B.Cu) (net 1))
 (segment (start 117.15 106.48) (end 120.93 106.48) (width 0.349) (layer B.Cu) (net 1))
 (segment (start 134.93 105.98) (end 135.97 107.02) (width 0.349) (layer B.Cu) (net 5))
 (segment (start 117.15 105.98) (end 134.93 105.98) (width 0.349) (layer B.Cu) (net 5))
 (segment (start 145.67 107.02) (end 145.77 107.12) (width 0.349) (layer B.Cu) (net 5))
 (segment (start 143.92 107.02) (end 145.67 107.02) (width 0.349) (layer B.Cu) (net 5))
 (segment (start 159.42 107.02) (end 161.3075 107.02) (width 0.349) (layer B.Cu) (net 4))
 (segment (start 157.88 105.48) (end 159.42 107.02) (width 0.349) (layer B.Cu) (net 4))
 (segment (start 149.68 105.48) (end 157.88 105.48) (width 0.349) (layer B.Cu) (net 4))
 (segment (start 117.15 105.48) (end 149.68 105.48) (width 0.349) (layer B.Cu) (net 4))
 (segment (start 149.68 105.48) (end 149.93 105.48) (width 0.349) (layer B.Cu) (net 4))
 (segment (start 165.4175 104.98) (end 165.57 105.1325) (width 0.349) (layer B.Cu) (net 3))
 (segment (start 117.15 104.98) (end 165.4175 104.98) (width 0.349) (layer B.Cu) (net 3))
 (segment (start 165.57 105.1325) (end 166.8625 105.1325) (width 0.349) (layer B.Cu) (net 3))
 (segment (start 168.2 106.47) (end 168.695 106.47) (width 0.349) (layer B.Cu) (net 3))
 (segment (start 166.8625 105.1325) (end 168.2 106.47) (width 0.349) (layer B.Cu) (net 3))
 (segment (start 168.7 106.47) (end 172.37 106.47) (width 0.75) (layer B.Cu) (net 3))
 (segment (start 126.3725 100.04) (end 127.9975 100.04) (width 0.349) (layer B.Cu) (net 10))
 (segment (start 140.875 100.04) (end 142.4375 100.04) (width 0.349) (layer B.Cu) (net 8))
 (segment (start 156.3925 100.02) (end 158.0175 100.02) (width 0.349) (layer B.Cu) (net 6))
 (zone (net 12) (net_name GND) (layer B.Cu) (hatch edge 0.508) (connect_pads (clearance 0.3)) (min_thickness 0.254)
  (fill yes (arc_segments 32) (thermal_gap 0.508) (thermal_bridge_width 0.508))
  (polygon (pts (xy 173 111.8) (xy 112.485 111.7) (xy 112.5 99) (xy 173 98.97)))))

